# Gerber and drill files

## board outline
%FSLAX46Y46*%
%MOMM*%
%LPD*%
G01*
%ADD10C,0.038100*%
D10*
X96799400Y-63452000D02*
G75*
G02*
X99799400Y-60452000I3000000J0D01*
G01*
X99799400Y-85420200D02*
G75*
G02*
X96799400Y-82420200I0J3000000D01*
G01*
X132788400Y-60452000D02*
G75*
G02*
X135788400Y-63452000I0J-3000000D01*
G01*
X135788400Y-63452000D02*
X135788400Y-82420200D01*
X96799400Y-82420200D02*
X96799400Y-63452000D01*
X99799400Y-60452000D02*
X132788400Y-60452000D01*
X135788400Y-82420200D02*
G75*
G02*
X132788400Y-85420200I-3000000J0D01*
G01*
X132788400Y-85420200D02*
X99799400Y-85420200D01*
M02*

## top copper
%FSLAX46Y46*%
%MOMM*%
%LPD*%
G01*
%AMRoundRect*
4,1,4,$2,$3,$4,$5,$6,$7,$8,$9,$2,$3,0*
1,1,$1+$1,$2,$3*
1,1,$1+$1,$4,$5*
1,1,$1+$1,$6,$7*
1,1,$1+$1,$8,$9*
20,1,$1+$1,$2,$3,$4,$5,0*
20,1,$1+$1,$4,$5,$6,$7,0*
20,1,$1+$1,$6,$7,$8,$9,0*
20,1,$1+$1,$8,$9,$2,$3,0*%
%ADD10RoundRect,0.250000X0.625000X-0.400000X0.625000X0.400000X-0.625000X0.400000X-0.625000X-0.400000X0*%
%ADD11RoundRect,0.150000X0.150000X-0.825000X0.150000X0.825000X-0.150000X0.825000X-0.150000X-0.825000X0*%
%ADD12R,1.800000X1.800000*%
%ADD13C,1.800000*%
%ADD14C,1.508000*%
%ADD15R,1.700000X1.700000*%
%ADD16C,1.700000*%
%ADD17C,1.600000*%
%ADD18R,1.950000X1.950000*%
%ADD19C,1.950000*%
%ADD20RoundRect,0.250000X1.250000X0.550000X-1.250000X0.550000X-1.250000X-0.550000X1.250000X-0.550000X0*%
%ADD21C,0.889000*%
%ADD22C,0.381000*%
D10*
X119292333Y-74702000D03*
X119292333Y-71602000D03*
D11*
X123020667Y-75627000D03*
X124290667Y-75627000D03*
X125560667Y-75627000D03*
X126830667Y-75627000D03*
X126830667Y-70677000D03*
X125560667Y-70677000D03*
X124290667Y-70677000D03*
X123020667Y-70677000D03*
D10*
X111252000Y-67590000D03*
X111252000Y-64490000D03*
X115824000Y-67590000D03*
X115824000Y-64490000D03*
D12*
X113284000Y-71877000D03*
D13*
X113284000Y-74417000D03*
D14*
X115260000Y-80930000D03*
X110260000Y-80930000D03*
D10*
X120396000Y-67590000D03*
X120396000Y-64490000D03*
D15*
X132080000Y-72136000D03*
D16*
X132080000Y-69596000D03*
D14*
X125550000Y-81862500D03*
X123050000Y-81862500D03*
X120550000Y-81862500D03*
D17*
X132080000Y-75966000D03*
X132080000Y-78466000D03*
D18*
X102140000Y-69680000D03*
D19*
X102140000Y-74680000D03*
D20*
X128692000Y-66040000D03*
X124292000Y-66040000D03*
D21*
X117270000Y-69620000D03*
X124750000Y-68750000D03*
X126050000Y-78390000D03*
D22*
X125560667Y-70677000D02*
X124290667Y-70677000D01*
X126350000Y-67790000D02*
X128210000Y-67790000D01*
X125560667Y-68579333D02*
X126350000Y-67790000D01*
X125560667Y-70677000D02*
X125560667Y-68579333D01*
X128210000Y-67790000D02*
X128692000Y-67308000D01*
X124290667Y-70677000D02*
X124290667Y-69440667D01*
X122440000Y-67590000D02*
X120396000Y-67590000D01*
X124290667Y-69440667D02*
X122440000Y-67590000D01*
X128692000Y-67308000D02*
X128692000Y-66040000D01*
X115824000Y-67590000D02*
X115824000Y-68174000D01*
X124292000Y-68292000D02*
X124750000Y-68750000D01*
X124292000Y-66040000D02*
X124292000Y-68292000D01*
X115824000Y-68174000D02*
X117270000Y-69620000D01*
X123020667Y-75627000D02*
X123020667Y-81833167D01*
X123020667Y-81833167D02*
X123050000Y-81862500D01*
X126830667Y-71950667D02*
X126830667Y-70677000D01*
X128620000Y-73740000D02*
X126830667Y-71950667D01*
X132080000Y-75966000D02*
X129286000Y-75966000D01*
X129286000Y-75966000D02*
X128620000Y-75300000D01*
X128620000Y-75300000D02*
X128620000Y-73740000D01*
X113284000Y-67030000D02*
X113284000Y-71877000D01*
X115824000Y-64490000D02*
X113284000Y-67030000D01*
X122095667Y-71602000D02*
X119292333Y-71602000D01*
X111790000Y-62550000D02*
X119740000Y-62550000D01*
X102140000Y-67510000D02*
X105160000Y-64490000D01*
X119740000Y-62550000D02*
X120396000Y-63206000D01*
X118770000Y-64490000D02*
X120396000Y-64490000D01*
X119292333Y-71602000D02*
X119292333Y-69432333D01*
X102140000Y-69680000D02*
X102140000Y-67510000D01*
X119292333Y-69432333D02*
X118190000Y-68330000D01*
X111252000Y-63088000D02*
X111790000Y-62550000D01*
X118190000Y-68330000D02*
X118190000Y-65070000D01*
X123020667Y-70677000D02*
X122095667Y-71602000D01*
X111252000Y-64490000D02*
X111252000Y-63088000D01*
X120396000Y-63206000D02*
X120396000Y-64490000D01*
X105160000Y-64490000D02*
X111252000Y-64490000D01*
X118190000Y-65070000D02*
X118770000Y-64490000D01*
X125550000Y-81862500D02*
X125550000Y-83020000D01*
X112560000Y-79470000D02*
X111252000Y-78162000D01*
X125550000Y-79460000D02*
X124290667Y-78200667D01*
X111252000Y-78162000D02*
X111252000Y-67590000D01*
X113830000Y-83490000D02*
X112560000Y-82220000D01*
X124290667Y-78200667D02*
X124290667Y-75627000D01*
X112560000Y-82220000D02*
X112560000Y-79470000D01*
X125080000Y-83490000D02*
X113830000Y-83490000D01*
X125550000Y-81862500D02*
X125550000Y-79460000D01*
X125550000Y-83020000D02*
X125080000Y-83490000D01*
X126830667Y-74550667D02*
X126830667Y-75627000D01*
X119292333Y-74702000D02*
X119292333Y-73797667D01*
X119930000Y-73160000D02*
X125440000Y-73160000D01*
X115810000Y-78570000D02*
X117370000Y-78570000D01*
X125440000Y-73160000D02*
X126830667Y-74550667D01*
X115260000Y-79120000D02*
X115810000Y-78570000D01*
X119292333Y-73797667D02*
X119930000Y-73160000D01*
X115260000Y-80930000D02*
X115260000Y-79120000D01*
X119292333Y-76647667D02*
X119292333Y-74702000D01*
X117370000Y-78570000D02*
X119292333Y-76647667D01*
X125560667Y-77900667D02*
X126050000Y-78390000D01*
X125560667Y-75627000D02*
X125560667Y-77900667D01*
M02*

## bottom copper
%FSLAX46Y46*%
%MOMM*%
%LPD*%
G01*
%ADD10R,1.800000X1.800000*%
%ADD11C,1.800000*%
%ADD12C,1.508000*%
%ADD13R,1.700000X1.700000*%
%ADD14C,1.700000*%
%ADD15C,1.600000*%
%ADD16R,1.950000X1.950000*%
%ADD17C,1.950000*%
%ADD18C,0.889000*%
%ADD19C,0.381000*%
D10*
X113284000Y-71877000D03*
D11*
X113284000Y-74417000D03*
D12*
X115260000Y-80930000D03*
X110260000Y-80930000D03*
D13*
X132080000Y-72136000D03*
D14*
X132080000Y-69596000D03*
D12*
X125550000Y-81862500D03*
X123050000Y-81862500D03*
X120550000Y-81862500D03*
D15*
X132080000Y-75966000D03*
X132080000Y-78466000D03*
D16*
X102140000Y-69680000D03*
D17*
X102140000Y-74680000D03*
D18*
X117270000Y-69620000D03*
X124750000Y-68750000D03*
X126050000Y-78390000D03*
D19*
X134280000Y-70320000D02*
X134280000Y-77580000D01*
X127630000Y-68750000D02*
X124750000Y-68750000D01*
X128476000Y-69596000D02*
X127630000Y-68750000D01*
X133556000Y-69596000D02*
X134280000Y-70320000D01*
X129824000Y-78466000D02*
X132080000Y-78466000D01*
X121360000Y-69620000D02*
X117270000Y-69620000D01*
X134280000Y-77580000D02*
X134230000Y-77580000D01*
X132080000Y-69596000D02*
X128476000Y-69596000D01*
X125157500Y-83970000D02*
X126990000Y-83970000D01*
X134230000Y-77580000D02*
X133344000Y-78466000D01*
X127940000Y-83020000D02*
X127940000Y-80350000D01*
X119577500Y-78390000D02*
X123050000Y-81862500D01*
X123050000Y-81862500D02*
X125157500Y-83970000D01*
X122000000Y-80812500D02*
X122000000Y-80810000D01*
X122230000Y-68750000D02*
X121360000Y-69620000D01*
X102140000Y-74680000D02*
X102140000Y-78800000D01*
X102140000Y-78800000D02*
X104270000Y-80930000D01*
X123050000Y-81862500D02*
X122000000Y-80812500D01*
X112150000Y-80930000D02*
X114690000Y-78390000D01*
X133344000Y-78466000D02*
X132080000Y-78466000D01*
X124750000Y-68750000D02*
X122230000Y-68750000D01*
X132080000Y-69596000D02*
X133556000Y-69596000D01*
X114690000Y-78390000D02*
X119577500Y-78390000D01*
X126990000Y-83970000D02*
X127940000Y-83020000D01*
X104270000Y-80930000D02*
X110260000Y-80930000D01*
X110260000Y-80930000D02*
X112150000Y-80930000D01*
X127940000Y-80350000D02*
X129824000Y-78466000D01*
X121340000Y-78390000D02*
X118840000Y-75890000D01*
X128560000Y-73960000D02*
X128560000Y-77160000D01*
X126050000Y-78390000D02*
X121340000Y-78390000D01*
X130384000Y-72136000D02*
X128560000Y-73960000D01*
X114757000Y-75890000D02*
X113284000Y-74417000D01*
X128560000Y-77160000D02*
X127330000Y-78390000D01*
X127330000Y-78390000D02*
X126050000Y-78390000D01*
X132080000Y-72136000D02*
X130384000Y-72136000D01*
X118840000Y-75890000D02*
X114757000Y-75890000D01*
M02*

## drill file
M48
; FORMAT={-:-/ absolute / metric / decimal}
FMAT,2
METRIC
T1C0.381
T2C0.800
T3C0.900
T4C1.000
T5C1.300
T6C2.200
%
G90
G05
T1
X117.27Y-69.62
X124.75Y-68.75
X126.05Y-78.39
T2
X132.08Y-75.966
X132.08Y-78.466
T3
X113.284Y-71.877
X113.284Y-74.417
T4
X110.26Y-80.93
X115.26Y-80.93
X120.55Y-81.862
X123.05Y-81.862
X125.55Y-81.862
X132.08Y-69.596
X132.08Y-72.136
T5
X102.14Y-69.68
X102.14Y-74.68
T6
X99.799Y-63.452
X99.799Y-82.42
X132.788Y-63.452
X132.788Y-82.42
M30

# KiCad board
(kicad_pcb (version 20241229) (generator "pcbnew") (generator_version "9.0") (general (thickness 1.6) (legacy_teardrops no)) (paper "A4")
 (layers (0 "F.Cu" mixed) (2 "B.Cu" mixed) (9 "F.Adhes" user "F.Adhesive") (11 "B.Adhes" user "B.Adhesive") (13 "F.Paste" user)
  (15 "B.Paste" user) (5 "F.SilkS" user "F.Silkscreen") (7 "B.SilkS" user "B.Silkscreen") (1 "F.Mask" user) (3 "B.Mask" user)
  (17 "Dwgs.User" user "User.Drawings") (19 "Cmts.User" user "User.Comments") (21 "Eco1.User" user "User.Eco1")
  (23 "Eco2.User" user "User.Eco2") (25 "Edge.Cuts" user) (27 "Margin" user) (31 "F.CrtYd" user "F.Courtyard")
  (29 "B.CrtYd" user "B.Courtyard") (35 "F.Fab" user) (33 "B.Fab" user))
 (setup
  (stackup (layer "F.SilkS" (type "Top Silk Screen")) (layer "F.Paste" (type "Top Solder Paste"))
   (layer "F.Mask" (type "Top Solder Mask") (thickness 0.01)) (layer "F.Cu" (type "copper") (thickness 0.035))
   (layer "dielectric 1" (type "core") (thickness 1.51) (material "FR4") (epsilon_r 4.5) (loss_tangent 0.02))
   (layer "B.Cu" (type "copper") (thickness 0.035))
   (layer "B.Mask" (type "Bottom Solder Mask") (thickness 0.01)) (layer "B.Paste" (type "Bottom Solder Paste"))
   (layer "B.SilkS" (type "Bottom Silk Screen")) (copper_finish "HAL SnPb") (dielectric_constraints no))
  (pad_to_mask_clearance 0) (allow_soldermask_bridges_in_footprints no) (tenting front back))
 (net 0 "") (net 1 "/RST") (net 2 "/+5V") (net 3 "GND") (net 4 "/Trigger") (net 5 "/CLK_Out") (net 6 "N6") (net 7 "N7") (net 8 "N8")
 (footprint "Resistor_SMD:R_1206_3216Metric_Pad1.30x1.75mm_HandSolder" (layer "F.Cu") (at 119.292333 73.152 90)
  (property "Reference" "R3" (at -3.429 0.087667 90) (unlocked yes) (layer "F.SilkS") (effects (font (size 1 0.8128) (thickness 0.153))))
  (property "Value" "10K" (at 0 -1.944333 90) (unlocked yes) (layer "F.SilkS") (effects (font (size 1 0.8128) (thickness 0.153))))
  (pad "1" smd roundrect (at -1.55 0 90) (size 1.3 1.75) (layers "F.Cu" "F.Mask" "F.Paste") (roundrect_rratio 0.192308) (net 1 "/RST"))
  (pad "2" smd roundrect (at 1.55 0 90) (size 1.3 1.75) (layers "F.Cu" "F.Mask" "F.Paste") (roundrect_rratio 0.192308) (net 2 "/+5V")))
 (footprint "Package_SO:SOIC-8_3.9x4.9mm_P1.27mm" (layer "F.Cu") (at 124.925667 73.152 90)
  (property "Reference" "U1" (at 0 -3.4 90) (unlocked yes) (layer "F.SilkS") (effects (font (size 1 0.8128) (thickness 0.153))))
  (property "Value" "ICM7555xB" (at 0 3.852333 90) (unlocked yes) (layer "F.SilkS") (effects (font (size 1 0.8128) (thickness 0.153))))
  (pad "1" smd roundrect (at -2.475 -1.905 90) (size 1.95 0.6) (layers "F.Cu" "F.Mask" "F.Paste") (roundrect_rratio 0.25) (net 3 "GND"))
  (pad "2" smd roundrect (at -2.475 -0.635 90) (size 1.95 0.6) (layers "F.Cu" "F.Mask" "F.Paste") (roundrect_rratio 0.25) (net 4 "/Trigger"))
  (pad "3" smd roundrect (at -2.475 0.635 90) (size 1.95 0.6) (layers "F.Cu" "F.Mask" "F.Paste") (roundrect_rratio 0.25) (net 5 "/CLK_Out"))
  (pad "4" smd roundrect (at -2.475 1.905 90) (size 1.95 0.6) (layers "F.Cu" "F.Mask" "F.Paste") (roundrect_rratio 0.25) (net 1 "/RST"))
  (pad "5" smd roundrect (at 2.475 1.905 90) (size 1.95 0.6) (layers "F.Cu" "F.Mask" "F.Paste") (roundrect_rratio 0.25) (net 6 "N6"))
  (pad "6" smd roundrect (at 2.475 0.635 90) (size 1.95 0.6) (layers "F.Cu" "F.Mask" "F.Paste") (roundrect_rratio 0.25) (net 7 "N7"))
  (pad "7" smd roundrect (at 2.475 -0.635 90) (size 1.95 0.6) (layers "F.Cu" "F.Mask" "F.Paste") (roundrect_rratio 0.25) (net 7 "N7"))
  (pad "8" smd roundrect (at 2.475 -1.905 90) (size 1.95 0.6) (layers "F.Cu" "F.Mask" "F.Paste") (roundrect_rratio 0.25) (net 2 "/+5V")))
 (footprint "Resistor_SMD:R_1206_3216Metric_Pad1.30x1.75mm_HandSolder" (layer "F.Cu") (at 111.252 66.04 90)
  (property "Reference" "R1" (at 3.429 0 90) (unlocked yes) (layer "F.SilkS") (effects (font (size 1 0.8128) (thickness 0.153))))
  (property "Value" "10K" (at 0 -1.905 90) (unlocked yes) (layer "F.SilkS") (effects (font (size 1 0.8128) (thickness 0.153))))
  (pad "1" smd roundrect (at -1.55 0 90) (size 1.3 1.75) (layers "F.Cu" "F.Mask" "F.Paste") (roundrect_rratio 0.192308) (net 4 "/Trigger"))
  (pad "2" smd roundrect (at 1.55 0 90) (size 1.3 1.75) (layers "F.Cu" "F.Mask" "F.Paste") (roundrect_rratio 0.192308) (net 2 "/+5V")))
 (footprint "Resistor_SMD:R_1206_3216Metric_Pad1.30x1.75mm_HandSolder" (layer "F.Cu") (at 115.824 66.04 90)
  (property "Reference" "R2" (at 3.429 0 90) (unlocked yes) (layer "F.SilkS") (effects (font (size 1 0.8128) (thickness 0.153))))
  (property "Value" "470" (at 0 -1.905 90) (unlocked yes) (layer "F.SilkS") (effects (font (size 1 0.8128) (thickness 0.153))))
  (pad "1" smd roundrect (at -1.55 0 90) (size 1.3 1.75) (layers "F.Cu" "F.Mask" "F.Paste") (roundrect_rratio 0.192308) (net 3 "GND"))
  (pad "2" smd roundrect (at 1.55 0 90) (size 1.3 1.75) (layers "F.Cu" "F.Mask" "F.Paste") (roundrect_rratio 0.192308) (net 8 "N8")))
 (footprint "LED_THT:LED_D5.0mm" (layer "F.Cu") (at 113.284 71.877 -90)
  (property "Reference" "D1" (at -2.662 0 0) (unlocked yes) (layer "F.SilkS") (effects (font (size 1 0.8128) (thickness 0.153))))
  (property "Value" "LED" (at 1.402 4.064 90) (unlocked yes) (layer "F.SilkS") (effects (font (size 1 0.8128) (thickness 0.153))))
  (pad "1" thru_hole rect (at 0 0 270) (size 1.8 1.8) (drill 0.9) (layers "*.Cu" "*.Mask") (remove_unused_layers no) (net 8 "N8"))
  (pad "2" thru_hole circle (at 2.54 0 270) (size 1.8 1.8) (drill 0.9) (layers "*.Cu" "*.Mask") (remove_unused_layers no) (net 5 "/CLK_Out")))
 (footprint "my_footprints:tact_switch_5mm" (layer "F.Cu") (at 112.76 80.93 180)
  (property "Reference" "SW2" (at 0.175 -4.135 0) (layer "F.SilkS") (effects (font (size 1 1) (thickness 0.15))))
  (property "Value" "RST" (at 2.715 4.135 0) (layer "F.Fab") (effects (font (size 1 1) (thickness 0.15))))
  (pad "1" thru_hole circle (at -2.5 0 180) (size 1.508 1.508) (drill 1) (layers "*.Cu" "*.Mask") (remove_unused_layers no) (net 1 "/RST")
   (solder_mask_margin 0.102))
  (pad "2" thru_hole circle (at 2.5 0 180) (size 1.508 1.508) (drill 1) (layers "*.Cu" "*.Mask") (remove_unused_layers no) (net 3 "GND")
   (solder_mask_margin 0.102)))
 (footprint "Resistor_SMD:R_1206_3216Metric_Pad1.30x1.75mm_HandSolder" (layer "F.Cu") (at 120.396 66.04 90)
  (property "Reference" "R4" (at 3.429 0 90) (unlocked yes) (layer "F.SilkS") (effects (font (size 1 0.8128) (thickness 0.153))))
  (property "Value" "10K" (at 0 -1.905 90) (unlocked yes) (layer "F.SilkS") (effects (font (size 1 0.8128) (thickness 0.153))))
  (pad "1" smd roundrect (at -1.55 0 90) (size 1.3 1.75) (layers "F.Cu" "F.Mask" "F.Paste") (roundrect_rratio 0.192308) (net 7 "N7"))
  (pad "2" smd roundrect (at 1.55 0 90) (size 1.3 1.75) (layers "F.Cu" "F.Mask" "F.Paste") (roundrect_rratio 0.192308) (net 2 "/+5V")))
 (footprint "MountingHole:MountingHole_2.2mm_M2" (layer "F.Cu") (at 99.7994 63.452)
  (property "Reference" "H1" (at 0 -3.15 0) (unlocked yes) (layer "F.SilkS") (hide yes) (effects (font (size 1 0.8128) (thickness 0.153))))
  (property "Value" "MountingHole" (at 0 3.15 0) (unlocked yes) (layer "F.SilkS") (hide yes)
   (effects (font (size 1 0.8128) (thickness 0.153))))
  (pad "" np_thru_hole circle (at 0 0) (size 2.2 2.2) (drill 2.2) (layers "*.Cu" "*.Mask")))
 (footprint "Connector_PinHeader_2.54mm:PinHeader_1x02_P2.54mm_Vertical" (layer "F.Cu") (at 132.08 72.136 180)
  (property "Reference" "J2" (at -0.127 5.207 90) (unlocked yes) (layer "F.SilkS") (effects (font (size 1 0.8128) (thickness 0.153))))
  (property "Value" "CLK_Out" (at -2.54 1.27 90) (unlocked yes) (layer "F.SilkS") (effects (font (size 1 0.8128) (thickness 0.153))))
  (pad "1" thru_hole rect (at 0 0 180) (size 1.7 1.7) (drill 1) (layers "*.Cu" "*.Mask") (remove_unused_layers no) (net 5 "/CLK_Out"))
  (pad "2" thru_hole circle (at 0 2.54 180) (size 1.7 1.7) (drill 1) (layers "*.Cu" "*.Mask") (remove_unused_layers no) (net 3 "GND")))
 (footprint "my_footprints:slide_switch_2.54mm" (layer "F.Cu") (at 123.05 81.8625 180)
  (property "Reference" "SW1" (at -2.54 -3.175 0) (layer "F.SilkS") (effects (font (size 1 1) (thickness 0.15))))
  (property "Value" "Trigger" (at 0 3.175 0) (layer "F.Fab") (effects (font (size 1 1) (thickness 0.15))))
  (pad "1" thru_hole circle (at -2.5 0 180) (size 1.508 1.508) (drill 1) (layers "*.Cu" "*.Mask") (remove_unused_layers no)
   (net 4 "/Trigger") (solder_mask_margin 0.102))
  (pad "2" thru_hole circle (at 0 0 180) (size 1.508 1.508) (drill 1) (layers "*.Cu" "*.Mask") (remove_unused_layers no) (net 3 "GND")
   (solder_mask_margin 0.102))
  (pad "3" thru_hole circle (at 2.5 0 180) (size 1.508 1.508) (drill 1) (layers "*.Cu" "*.Mask") (remove_unused_layers no)
   (solder_mask_margin 0.102)))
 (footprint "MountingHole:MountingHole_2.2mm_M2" (layer "F.Cu") (at 132.7884 82.4202)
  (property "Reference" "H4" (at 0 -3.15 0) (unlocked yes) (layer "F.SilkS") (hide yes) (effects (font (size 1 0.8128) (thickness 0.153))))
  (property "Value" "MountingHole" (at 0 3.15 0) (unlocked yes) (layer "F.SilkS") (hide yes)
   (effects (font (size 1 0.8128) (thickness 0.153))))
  (pad "" np_thru_hole circle (at 0 0) (size 2.2 2.2) (drill 2.2) (layers "*.Cu" "*.Mask")))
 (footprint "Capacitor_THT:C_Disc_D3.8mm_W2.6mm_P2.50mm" (layer "F.Cu") (at 132.08 75.966 -90)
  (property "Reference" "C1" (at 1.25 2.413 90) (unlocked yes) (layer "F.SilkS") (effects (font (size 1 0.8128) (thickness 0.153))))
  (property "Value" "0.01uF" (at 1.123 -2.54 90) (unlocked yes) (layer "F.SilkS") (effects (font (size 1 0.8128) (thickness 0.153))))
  (pad "1" thru_hole circle (at 0 0 270) (size 1.6 1.6) (drill 0.8) (layers "*.Cu" "*.Mask") (remove_unused_layers no) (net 6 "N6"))
  (pad "2" thru_hole circle (at 2.5 0 270) (size 1.6 1.6) (drill 0.8) (layers "*.Cu" "*.Mask") (remove_unused_layers no) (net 3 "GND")))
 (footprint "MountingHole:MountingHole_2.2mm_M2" (layer "F.Cu") (at 132.7884 63.452)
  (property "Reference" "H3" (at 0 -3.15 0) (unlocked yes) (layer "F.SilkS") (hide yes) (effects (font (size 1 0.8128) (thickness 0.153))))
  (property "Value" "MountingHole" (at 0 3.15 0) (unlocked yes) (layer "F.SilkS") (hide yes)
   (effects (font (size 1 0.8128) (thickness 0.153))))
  (pad "" np_thru_hole circle (at 0 0) (size 2.2 2.2) (drill 2.2) (layers "*.Cu" "*.Mask")))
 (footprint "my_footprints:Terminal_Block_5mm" (layer "F.Cu") (at 102.14 72.18 -90)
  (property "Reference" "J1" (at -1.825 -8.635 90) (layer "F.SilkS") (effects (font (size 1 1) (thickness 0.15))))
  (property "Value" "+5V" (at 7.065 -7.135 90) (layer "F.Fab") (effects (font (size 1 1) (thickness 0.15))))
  (pad "1" thru_hole rect (at -2.5 0 270) (size 1.95 1.95) (drill 1.3) (layers "*.Cu" "*.Mask") (remove_unused_layers no) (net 2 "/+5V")
   (solder_mask_margin 0.102))
  (pad "2" thru_hole circle (at 2.5 0 270) (size 1.95 1.95) (drill 1.3) (layers "*.Cu" "*.Mask") (remove_unused_layers no) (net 3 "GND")
   (solder_mask_margin 0.102)))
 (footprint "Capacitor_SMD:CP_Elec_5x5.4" (layer "F.Cu") (at 126.492 66.04 180)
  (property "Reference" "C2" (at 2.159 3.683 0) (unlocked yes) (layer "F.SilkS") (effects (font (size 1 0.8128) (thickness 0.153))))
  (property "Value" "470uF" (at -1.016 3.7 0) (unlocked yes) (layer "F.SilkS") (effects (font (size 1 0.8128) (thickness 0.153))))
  (pad "1" smd roundrect (at -2.2 0 180) (size 3 1.6) (layers "F.Cu" "F.Mask" "F.Paste") (roundrect_rratio 0.15625) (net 7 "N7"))
  (pad "2" smd roundrect (at 2.2 0 180) (size 3 1.6) (layers "F.Cu" "F.Mask" "F.Paste") (roundrect_rratio 0.15625) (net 3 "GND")))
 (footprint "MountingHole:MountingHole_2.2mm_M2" (layer "F.Cu") (at 99.7994 82.4202)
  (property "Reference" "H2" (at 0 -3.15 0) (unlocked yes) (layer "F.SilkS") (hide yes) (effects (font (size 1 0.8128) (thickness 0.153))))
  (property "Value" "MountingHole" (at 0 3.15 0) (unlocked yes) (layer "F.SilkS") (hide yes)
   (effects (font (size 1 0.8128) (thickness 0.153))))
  (pad "" np_thru_hole circle (at 0 0) (size 2.2 2.2) (drill 2.2) (layers "*.Cu" "*.Mask")))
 (gr_arc (start 96.7994 63.452) (mid 97.67808 61.33068) (end 99.7994 60.452) (stroke (width 0.0381) (type default)) (layer "Edge.Cuts"))
 (gr_arc (start 99.7994 85.4202) (mid 97.67808 84.54152) (end 96.7994 82.4202) (stroke (width 0.0381) (type default)) (layer "Edge.Cuts"))
 (gr_arc (start 132.7884 60.452) (mid 134.90972 61.33068) (end 135.7884 63.452) (stroke (width 0.0381) (type default)) (layer "Edge.Cuts"))
 (gr_line (start 135.7884 63.452) (end 135.7884 82.4202) (stroke (width 0.0381) (type default)) (layer "Edge.Cuts"))
 (gr_line (start 96.7994 82.4202) (end 96.7994 63.452) (stroke (width 0.0381) (type default)) (layer "Edge.Cuts"))
 (gr_line (start 99.7994 60.452) (end 132.7884 60.452) (stroke (width 0.0381) (type default)) (layer "Edge.Cuts"))
 (gr_arc (start 135.7884 82.4202) (mid 134.90972 84.54152) (end 132.7884 85.4202) (stroke (width 0.0381) (type default)) (layer "Edge.Cuts"))
 (gr_line (start 132.7884 85.4202) (end 99.7994 85.4202) (stroke (width 0.0381) (type default)) (layer "Edge.Cuts"))
 (segment (start 125.560667 70.677) (end 124.290667 70.677) (width 0.381) (layer "F.Cu") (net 7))
 (segment (start 126.35 67.79) (end 128.21 67.79) (width 0.381) (layer "F.Cu") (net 7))
 (segment (start 125.560667 68.579333) (end 126.35 67.79) (width 0.381) (layer "F.Cu") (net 7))
 (segment (start 125.560667 70.677) (end 125.560667 68.579333) (width 0.381) (layer "F.Cu") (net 7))
 (segment (start 128.21 67.79) (end 128.692 67.308) (width 0.381) (layer "F.Cu") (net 7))
 (segment (start 124.290667 70.677) (end 124.290667 69.440667) (width 0.381) (layer "F.Cu") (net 7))
 (segment (start 122.44 67.59) (end 120.396 67.59) (width 0.381) (layer "F.Cu") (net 7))
 (segment (start 124.290667 69.440667) (end 122.44 67.59) (width 0.381) (layer "F.Cu") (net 7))
 (segment (start 128.692 67.308) (end 128.692 66.04) (width 0.381) (layer "F.Cu") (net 7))
 (segment (start 115.824 67.59) (end 115.824 68.174) (width 0.381) (layer "F.Cu") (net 3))
 (segment (start 124.292 68.292) (end 124.75 68.75) (width 0.381) (layer "F.Cu") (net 3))
 (segment (start 124.292 66.04) (end 124.292 68.292) (width 0.381) (layer "F.Cu") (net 3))
 (segment (start 115.824 68.174) (end 117.27 69.62) (width 0.381) (layer "F.Cu") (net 3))
 (segment (start 123.020667 75.627) (end 123.020667 81.833167) (width 0.381) (layer "F.Cu") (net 3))
 (segment (start 123.020667 81.833167) (end 123.05 81.8625) (width 0.381) (layer "F.Cu") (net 3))
 (via (at 117.27 69.62) (size 0.889) (drill 0.381) (layers "F.Cu" "B.Cu") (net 3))
 (via (at 124.75 68.75) (size 0.889) (drill 0.381) (layers "F.Cu" "B.Cu") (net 3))
 (segment (start 134.28 70.32) (end 134.28 77.58) (width 0.381) (layer "B.Cu") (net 3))
 (segment (start 127.63 68.75) (end 124.75 68.75) (width 0.381) (layer "B.Cu") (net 3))
 (segment (start 128.476 69.596) (end 127.63 68.75) (width 0.381) (layer "B.Cu") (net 3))
 (segment (start 133.556 69.596) (end 134.28 70.32) (width 0.381) (layer "B.Cu") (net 3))
 (segment (start 129.824 78.466) (end 132.08 78.466) (width 0.381) (layer "B.Cu") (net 3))
 (segment (start 121.36 69.62) (end 117.27 69.62) (width 0.381) (layer "B.Cu") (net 3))
 (segment (start 134.28 77.58) (end 134.23 77.58) (width 0.381) (layer "B.Cu") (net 3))
 (segment (start 132.08 69.596) (end 128.476 69.596) (width 0.381) (layer "B.Cu") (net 3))
 (segment (start 125.1575 83.97) (end 126.99 83.97) (width 0.381) (layer "B.Cu") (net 3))
 (segment (start 134.23 77.58) (end 133.344 78.466) (width 0.381) (layer "B.Cu") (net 3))
 (segment (start 127.94 83.02) (end 127.94 80.35) (width 0.381) (layer "B.Cu") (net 3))
 (segment (start 119.5775 78.39) (end 123.05 81.8625) (width 0.381) (layer "B.Cu") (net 3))
 (segment (start 123.05 81.8625) (end 125.1575 83.97) (width 0.381) (layer "B.Cu") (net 3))
 (segment (start 122 80.8125) (end 122 80.81) (width 0.381) (layer "B.Cu") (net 3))
 (segment (start 122.23 68.75) (end 121.36 69.62) (width 0.381) (layer "B.Cu") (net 3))
 (segment (start 102.14 74.68) (end 102.14 78.8) (width 0.381) (layer "B.Cu") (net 3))
 (segment (start 102.14 78.8) (end 104.27 80.93) (width 0.381) (layer "B.Cu") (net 3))
 (segment (start 123.05 81.8625) (end 122 80.8125) (width 0.381) (layer "B.Cu") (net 3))
 (segment (start 112.15 80.93) (end 114.69 78.39) (width 0.381) (layer "B.Cu") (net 3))
 (segment (start 133.344 78.466) (end 132.08 78.466) (width 0.381) (layer "B.Cu") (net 3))
 (segment (start 124.75 68.75) (end 122.23 68.75) (width 0.381) (layer "B.Cu") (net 3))
 (segment (start 132.08 69.596) (end 133.556 69.596) (width 0.381) (layer "B.Cu") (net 3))
 (segment (start 114.69 78.39) (end 119.5775 78.39) (width 0.381) (layer "B.Cu") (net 3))
 (segment (start 126.99 83.97) (end 127.94 83.02) (width 0.381) (layer "B.Cu") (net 3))
 (segment (start 104.27 80.93) (end 110.26 80.93) (width 0.381) (layer "B.Cu") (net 3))
 (segment (start 110.26 80.93) (end 112.15 80.93) (width 0.381) (layer "B.Cu") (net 3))
 (segment (start 127.94 80.35) (end 129.824 78.466) (width 0.381) (layer "B.Cu") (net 3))
 (segment (start 126.830667 71.950667) (end 126.830667 70.677) (width 0.381) (layer "F.Cu") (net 6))
 (segment (start 128.62 73.74) (end 126.830667 71.950667) (width 0.381) (layer "F.Cu") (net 6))
 (segment (start 132.08 75.966) (end 129.286 75.966) (width 0.381) (layer "F.Cu") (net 6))
 (segment (start 129.286 75.966) (end 128.62 75.3) (width 0.381) (layer "F.Cu") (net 6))
 (segment (start 128.62 75.3) (end 128.62 73.74) (width 0.381) (layer "F.Cu") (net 6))
 (segment (start 113.284 67.03) (end 113.284 71.877) (width 0.381) (layer "F.Cu") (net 8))
 (segment (start 115.824 64.49) (end 113.284 67.03) (width 0.381) (layer "F.Cu") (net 8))
 (segment (start 122.095667 71.602) (end 119.292333 71.602) (width 0.381) (layer "F.Cu") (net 2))
 (segment (start 111.79 62.55) (end 119.74 62.55) (width 0.381) (layer "F.Cu") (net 2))
 (segment (start 102.14 67.51) (end 105.16 64.49) (width 0.381) (layer "F.Cu") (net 2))
 (segment (start 119.74 62.55) (end 120.396 63.206) (width 0.381) (layer "F.Cu") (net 2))
 (segment (start 118.77 64.49) (end 120.396 64.49) (width 0.381) (layer "F.Cu") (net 2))
 (segment (start 119.292333 71.602) (end 119.292333 69.432333) (width 0.381) (layer "F.Cu") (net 2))
 (segment (start 102.14 69.68) (end 102.14 67.51) (width 0.381) (layer "F.Cu") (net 2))
 (segment (start 119.292333 69.432333) (end 118.19 68.33) (width 0.381) (layer "F.Cu") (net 2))
 (segment (start 111.252 63.088) (end 111.79 62.55) (width 0.381) (layer "F.Cu") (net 2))
 (segment (start 118.19 68.33) (end 118.19 65.07) (width 0.381) (layer "F.Cu") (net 2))
 (segment (start 123.020667 70.677) (end 122.095667 71.602) (width 0.381) (layer "F.Cu") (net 2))
 (segment (start 111.252 64.49) (end 111.252 63.088) (width 0.381) (layer "F.Cu") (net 2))
 (segment (start 120.396 63.206) (end 120.396 64.49) (width 0.381) (layer "F.Cu") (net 2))
 (segment (start 105.16 64.49) (end 111.252 64.49) (width 0.381) (layer "F.Cu") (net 2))
 (segment (start 118.19 65.07) (end 118.77 64.49) (width 0.381) (layer "F.Cu") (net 2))
 (segment (start 125.55 81.8625) (end 125.55 83.02) (width 0.381) (layer "F.Cu") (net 4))
 (segment (start 112.56 79.47) (end 111.252 78.162) (width 0.381) (layer "F.Cu") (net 4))
 (segment (start 125.55 79.46) (end 124.290667 78.200667) (width 0.381) (layer "F.Cu") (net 4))
 (segment (start 111.252 78.162) (end 111.252 67.59) (width 0.381) (layer "F.Cu") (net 4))
 (segment (start 113.83 83.49) (end 112.56 82.22) (width 0.381) (layer "F.Cu") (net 4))
 (segment (start 124.290667 78.200667) (end 124.290667 75.627) (width 0.381) (layer "F.Cu") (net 4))
 (segment (start 112.56 82.22) (end 112.56 79.47) (width 0.381) (layer "F.Cu") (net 4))
 (segment (start 125.08 83.49) (end 113.83 83.49) (width 0.381) (layer "F.Cu") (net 4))
 (segment (start 125.55 81.8625) (end 125.55 79.46) (width 0.381) (layer "F.Cu") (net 4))
 (segment (start 125.55 83.02) (end 125.08 83.49) (width 0.381) (layer "F.Cu") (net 4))
 (segment (start 126.830667 74.550667) (end 126.830667 75.627) (width 0.381) (layer "F.Cu") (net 1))
 (segment (start 119.292333 74.702) (end 119.292333 73.797667) (width 0.381) (layer "F.Cu") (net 1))
 (segment (start 119.93 73.16) (end 125.44 73.16) (width 0.381) (layer "F.Cu") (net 1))
 (segment (start 115.81 78.57) (end 117.37 78.57) (width 0.381) (layer "F.Cu") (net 1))
 (segment (start 125.44 73.16) (end 126.830667 74.550667) (width 0.381) (layer "F.Cu") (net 1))
 (segment (start 115.26 79.12) (end 115.81 78.57) (width 0.381) (layer "F.Cu") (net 1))
 (segment (start 119.292333 73.797667) (end 119.93 73.16) (width 0.381) (layer "F.Cu") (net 1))
 (segment (start 115.26 80.93) (end 115.26 79.12) (width 0.381) (layer "F.Cu") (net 1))
 (segment (start 119.292333 76.647667) (end 119.292333 74.702) (width 0.381) (layer "F.Cu") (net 1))
 (segment (start 117.37 78.57) (end 119.292333 76.647667) (width 0.381) (layer "F.Cu") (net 1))
 (segment (start 125.560667 77.900667) (end 126.05 78.39) (width 0.381) (layer "F.Cu") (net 5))
 (segment (start 125.560667 75.627) (end 125.560667 77.900667) (width 0.381) (layer "F.Cu") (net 5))
 (via (at 126.05 78.39) (size 0.889) (drill 0.381) (layers "F.Cu" "B.Cu") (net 5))
 (segment (start 121.34 78.39) (end 118.84 75.89) (width 0.381) (layer "B.Cu") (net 5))
 (segment (start 128.56 73.96) (end 128.56 77.16) (width 0.381) (layer "B.Cu") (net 5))
 (segment (start 126.05 78.39) (end 121.34 78.39) (width 0.381) (layer "B.Cu") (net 5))
 (segment (start 130.384 72.136) (end 128.56 73.96) (width 0.381) (layer "B.Cu") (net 5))
 (segment (start 114.757 75.89) (end 113.284 74.417) (width 0.381) (layer "B.Cu") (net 5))
 (segment (start 128.56 77.16) (end 127.33 78.39) (width 0.381) (layer "B.Cu") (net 5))
 (segment (start 127.33 78.39) (end 126.05 78.39) (width 0.381) (layer "B.Cu") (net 5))
 (segment (start 132.08 72.136) (end 130.384 72.136) (width 0.381) (layer "B.Cu") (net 5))
 (segment (start 118.84 75.89) (end 114.757 75.89) (width 0.381) (layer "B.Cu") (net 5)))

